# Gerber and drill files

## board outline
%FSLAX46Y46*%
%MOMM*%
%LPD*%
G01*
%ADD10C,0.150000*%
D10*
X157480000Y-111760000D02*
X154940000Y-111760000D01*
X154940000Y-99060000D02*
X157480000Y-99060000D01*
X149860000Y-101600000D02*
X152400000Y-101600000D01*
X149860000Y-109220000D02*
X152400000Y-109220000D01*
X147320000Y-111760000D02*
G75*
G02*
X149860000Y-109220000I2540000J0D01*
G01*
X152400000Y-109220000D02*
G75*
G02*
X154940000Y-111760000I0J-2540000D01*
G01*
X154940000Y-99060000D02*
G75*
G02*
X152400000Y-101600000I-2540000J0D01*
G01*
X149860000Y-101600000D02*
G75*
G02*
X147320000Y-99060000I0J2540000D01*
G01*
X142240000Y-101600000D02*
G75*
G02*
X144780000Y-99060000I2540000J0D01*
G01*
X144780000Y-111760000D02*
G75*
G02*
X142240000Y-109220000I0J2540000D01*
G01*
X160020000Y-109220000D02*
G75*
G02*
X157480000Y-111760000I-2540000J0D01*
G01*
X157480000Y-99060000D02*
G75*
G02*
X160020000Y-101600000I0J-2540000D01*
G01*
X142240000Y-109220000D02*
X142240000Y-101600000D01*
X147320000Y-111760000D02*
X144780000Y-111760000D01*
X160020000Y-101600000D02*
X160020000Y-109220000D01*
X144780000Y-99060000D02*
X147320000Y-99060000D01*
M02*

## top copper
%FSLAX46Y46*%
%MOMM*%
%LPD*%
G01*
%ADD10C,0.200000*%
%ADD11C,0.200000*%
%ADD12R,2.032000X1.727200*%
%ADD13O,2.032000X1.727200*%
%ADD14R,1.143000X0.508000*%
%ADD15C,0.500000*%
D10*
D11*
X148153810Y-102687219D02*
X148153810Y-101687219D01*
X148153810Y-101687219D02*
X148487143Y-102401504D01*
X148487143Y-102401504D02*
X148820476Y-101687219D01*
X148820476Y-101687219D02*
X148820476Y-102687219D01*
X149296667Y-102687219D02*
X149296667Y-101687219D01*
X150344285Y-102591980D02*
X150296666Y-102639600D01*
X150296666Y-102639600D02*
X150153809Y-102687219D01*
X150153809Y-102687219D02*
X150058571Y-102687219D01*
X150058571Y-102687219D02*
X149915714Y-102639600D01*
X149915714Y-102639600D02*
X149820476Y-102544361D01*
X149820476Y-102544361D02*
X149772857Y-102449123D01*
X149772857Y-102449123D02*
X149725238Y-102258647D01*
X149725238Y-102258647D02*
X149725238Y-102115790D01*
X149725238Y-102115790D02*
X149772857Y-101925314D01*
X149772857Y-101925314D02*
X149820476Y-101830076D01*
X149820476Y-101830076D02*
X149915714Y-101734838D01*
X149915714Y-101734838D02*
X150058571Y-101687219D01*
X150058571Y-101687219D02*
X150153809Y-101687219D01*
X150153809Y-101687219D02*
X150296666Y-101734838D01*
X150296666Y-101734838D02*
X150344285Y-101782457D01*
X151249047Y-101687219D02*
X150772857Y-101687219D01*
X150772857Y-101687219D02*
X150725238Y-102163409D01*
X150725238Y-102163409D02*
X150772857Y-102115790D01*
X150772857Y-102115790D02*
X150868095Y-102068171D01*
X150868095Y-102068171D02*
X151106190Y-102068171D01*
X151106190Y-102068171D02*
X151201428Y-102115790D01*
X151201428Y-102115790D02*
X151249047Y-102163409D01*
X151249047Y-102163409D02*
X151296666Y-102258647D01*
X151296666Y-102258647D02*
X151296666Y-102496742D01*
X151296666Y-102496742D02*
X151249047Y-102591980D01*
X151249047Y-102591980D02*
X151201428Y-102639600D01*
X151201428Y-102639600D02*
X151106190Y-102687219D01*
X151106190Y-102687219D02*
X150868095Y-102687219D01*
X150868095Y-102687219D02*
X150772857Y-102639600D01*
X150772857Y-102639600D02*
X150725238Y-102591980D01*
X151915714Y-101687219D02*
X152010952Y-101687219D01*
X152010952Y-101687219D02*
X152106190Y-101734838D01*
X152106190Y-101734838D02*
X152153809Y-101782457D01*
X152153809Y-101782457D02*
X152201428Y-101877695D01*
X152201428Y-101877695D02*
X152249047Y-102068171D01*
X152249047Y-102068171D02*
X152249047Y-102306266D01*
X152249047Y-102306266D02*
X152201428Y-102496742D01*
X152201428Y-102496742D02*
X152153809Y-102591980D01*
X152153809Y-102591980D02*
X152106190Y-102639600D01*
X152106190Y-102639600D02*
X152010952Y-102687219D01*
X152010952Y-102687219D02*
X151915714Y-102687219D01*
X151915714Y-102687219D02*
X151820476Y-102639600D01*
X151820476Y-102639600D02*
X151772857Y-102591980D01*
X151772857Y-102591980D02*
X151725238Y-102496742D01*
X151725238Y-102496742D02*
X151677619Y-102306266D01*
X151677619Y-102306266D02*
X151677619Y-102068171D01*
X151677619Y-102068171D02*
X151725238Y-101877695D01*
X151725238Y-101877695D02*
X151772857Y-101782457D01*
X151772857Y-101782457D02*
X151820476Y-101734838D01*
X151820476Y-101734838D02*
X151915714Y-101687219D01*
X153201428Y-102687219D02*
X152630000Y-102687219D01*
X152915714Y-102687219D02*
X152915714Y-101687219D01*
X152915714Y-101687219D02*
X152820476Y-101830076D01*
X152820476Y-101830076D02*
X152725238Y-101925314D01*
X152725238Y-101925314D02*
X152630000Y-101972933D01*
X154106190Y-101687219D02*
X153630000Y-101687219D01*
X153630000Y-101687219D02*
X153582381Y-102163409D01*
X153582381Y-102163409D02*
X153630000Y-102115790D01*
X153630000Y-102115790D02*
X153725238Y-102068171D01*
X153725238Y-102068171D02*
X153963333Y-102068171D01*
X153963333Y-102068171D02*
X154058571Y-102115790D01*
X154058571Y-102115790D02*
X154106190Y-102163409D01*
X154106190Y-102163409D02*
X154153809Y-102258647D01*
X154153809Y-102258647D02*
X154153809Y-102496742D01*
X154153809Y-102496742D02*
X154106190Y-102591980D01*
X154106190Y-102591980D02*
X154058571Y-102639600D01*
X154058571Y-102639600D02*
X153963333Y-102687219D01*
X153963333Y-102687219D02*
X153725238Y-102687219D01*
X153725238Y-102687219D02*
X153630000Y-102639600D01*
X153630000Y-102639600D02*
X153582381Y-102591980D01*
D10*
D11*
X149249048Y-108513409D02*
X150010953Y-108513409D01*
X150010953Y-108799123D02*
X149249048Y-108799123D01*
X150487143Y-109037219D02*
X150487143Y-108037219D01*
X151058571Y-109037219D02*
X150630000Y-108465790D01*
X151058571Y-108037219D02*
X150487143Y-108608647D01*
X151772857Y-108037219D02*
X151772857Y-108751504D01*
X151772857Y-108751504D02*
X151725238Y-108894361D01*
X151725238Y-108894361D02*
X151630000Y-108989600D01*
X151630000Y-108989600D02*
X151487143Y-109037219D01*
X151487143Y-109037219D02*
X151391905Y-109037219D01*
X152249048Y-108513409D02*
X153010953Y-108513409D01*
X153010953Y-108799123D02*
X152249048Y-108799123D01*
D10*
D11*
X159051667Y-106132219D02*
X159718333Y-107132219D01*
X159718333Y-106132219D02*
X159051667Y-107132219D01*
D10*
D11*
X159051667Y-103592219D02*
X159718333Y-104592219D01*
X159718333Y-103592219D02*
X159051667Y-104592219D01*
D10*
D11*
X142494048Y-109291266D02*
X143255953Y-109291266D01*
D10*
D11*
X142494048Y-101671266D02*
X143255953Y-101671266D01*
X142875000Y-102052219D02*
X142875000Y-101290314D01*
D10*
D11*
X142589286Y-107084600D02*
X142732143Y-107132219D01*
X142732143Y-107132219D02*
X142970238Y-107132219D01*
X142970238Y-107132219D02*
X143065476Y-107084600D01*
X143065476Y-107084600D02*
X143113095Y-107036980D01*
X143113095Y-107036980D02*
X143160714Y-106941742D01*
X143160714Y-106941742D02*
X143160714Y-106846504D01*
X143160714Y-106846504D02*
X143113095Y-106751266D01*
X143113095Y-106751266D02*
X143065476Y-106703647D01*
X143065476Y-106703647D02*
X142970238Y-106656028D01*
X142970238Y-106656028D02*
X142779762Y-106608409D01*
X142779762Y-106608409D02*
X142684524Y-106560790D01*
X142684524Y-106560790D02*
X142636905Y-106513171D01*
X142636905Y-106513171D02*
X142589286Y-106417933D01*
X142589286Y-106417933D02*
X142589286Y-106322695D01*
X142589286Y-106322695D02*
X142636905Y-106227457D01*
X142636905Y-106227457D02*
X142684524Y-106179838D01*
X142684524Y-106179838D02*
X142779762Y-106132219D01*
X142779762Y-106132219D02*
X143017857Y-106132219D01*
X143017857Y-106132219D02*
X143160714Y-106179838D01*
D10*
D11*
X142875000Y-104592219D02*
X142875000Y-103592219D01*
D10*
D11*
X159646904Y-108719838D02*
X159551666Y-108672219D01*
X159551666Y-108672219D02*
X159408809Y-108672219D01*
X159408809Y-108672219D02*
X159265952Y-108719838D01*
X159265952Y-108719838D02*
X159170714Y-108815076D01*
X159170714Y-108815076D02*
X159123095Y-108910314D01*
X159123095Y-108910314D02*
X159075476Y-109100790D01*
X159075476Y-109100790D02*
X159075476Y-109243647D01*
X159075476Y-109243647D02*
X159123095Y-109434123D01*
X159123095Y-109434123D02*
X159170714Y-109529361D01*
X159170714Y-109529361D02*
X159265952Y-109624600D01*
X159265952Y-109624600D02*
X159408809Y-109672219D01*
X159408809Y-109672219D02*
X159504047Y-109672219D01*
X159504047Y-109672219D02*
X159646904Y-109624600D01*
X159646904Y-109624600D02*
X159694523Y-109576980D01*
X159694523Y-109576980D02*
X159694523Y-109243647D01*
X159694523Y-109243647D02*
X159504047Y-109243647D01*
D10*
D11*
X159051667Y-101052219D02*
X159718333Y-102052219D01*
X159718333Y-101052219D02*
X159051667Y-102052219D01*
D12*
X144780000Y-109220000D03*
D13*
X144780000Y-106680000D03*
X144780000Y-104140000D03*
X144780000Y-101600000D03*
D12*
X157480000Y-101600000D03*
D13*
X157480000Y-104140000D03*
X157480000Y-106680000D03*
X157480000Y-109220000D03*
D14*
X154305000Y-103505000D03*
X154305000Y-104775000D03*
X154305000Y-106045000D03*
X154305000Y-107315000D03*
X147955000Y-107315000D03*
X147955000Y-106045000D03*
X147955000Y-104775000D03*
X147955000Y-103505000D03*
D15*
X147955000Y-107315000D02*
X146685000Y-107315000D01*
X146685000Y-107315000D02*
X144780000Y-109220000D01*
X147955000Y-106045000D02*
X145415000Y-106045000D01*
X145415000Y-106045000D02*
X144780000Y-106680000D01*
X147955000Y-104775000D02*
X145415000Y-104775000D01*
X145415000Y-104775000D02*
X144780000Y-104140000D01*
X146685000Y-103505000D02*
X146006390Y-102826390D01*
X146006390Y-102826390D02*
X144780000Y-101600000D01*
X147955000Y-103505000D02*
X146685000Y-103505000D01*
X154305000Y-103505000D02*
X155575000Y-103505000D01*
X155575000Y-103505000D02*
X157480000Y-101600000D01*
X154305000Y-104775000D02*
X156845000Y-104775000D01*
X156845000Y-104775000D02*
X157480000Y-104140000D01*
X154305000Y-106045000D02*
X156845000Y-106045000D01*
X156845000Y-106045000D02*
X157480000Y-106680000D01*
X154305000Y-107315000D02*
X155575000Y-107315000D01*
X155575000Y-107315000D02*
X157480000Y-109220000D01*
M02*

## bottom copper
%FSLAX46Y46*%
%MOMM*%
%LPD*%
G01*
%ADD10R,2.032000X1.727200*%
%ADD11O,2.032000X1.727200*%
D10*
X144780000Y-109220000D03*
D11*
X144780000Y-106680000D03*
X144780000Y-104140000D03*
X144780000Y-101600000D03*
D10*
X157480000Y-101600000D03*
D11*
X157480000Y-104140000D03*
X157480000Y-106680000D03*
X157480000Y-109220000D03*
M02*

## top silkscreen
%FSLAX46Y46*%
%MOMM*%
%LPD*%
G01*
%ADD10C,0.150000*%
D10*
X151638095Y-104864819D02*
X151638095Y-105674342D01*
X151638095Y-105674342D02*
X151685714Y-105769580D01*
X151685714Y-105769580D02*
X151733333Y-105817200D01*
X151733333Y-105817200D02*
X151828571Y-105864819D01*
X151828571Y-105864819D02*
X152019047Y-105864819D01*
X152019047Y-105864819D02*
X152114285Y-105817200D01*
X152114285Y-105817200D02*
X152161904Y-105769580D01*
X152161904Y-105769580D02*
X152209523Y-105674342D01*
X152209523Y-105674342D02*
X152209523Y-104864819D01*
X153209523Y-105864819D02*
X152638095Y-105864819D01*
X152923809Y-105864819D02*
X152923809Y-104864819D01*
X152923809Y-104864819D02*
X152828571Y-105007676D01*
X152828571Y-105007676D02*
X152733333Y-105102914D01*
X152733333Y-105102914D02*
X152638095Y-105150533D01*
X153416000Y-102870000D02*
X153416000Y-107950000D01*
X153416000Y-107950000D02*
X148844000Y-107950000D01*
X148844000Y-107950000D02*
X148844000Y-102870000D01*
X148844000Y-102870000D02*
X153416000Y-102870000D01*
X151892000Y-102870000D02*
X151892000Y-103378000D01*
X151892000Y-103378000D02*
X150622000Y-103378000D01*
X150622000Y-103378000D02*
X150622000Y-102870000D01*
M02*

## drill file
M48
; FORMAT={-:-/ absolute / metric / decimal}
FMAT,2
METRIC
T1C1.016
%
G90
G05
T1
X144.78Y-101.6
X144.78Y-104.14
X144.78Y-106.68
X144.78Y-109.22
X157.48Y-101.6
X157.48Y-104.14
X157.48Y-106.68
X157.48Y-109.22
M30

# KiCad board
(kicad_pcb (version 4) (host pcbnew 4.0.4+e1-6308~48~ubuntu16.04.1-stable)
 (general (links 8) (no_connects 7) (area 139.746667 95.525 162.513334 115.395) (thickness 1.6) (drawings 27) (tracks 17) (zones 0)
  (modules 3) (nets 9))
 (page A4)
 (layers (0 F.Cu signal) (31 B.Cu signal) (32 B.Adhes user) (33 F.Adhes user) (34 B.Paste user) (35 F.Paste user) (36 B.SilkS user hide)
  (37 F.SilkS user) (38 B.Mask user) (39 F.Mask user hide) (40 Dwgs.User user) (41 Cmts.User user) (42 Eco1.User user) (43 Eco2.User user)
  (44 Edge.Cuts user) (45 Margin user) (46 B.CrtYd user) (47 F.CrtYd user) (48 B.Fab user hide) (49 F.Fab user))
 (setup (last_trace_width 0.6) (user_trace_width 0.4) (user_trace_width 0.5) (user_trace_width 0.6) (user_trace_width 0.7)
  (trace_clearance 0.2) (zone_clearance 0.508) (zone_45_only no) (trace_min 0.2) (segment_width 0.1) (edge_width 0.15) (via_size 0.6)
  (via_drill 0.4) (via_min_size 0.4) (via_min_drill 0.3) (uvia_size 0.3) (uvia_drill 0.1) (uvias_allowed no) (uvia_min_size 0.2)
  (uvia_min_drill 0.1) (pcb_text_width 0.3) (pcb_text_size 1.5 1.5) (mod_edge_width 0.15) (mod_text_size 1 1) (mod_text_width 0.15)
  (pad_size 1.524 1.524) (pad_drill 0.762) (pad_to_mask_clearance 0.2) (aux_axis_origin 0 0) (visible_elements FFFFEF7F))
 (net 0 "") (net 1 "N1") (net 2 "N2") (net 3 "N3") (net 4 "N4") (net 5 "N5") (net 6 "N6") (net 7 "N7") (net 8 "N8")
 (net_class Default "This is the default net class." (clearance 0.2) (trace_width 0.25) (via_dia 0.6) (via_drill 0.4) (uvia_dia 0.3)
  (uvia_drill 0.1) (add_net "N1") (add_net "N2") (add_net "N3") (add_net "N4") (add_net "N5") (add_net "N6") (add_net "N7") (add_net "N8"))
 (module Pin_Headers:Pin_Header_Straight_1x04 (layer B.Cu) (at 144.78 109.22)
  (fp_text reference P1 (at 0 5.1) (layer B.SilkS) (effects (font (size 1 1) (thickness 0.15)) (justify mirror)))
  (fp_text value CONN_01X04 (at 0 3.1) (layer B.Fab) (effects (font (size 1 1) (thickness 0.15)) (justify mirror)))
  (pad 1 thru_hole rect (at 0 0) (size 2.032 1.7272) (drill 1.016) (layers *.Cu *.Mask) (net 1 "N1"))
  (pad 2 thru_hole oval (at 0 -2.54) (size 2.032 1.7272) (drill 1.016) (layers *.Cu *.Mask) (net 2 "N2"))
  (pad 3 thru_hole oval (at 0 -5.08) (size 2.032 1.7272) (drill 1.016) (layers *.Cu *.Mask) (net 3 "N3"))
  (pad 4 thru_hole oval (at 0 -7.62) (size 2.032 1.7272) (drill 1.016) (layers *.Cu *.Mask) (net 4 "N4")))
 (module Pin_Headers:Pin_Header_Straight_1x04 (layer B.Cu) (at 157.48 101.6 180)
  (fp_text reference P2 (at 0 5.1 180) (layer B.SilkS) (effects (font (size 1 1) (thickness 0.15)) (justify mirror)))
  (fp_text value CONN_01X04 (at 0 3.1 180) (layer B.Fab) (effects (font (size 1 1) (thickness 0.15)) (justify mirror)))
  (pad 1 thru_hole rect (at 0 0 180) (size 2.032 1.7272) (drill 1.016) (layers *.Cu *.Mask) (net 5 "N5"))
  (pad 2 thru_hole oval (at 0 -2.54 180) (size 2.032 1.7272) (drill 1.016) (layers *.Cu *.Mask) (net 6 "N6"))
  (pad 3 thru_hole oval (at 0 -5.08 180) (size 2.032 1.7272) (drill 1.016) (layers *.Cu *.Mask) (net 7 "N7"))
  (pad 4 thru_hole oval (at 0 -7.62 180) (size 2.032 1.7272) (drill 1.016) (layers *.Cu *.Mask) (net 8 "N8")))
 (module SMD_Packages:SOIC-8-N (layer F.Cu) (at 151.13 105.41 270)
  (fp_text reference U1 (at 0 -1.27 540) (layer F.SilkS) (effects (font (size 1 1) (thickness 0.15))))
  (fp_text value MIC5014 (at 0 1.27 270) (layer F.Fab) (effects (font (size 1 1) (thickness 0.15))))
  (fp_line (start -2.54 -2.286) (end 2.54 -2.286) (layer F.SilkS) (width 0.15))
  (fp_line (start 2.54 -2.286) (end 2.54 2.286) (layer F.SilkS) (width 0.15))
  (fp_line (start 2.54 2.286) (end -2.54 2.286) (layer F.SilkS) (width 0.15))
  (fp_line (start -2.54 2.286) (end -2.54 -2.286) (layer F.SilkS) (width 0.15))
  (fp_line (start -2.54 -0.762) (end -2.032 -0.762) (layer F.SilkS) (width 0.15))
  (fp_line (start -2.032 -0.762) (end -2.032 0.508) (layer F.SilkS) (width 0.15))
  (fp_line (start -2.032 0.508) (end -2.54 0.508) (layer F.SilkS) (width 0.15))
  (pad 8 smd rect (at -1.905 -3.175 270) (size 0.508 1.143) (layers F.Cu F.Paste F.Mask) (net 5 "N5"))
  (pad 7 smd rect (at -0.635 -3.175 270) (size 0.508 1.143) (layers F.Cu F.Paste F.Mask) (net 6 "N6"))
  (pad 6 smd rect (at 0.635 -3.175 270) (size 0.508 1.143) (layers F.Cu F.Paste F.Mask) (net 7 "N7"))
  (pad 5 smd rect (at 1.905 -3.175 270) (size 0.508 1.143) (layers F.Cu F.Paste F.Mask) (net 8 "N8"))
  (pad 4 smd rect (at 1.905 3.175 270) (size 0.508 1.143) (layers F.Cu F.Paste F.Mask) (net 1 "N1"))
  (pad 3 smd rect (at 0.635 3.175 270) (size 0.508 1.143) (layers F.Cu F.Paste F.Mask) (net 2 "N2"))
  (pad 2 smd rect (at -0.635 3.175 270) (size 0.508 1.143) (layers F.Cu F.Paste F.Mask) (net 3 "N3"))
  (pad 1 smd rect (at -1.905 3.175 270) (size 0.508 1.143) (layers F.Cu F.Paste F.Mask) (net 4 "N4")))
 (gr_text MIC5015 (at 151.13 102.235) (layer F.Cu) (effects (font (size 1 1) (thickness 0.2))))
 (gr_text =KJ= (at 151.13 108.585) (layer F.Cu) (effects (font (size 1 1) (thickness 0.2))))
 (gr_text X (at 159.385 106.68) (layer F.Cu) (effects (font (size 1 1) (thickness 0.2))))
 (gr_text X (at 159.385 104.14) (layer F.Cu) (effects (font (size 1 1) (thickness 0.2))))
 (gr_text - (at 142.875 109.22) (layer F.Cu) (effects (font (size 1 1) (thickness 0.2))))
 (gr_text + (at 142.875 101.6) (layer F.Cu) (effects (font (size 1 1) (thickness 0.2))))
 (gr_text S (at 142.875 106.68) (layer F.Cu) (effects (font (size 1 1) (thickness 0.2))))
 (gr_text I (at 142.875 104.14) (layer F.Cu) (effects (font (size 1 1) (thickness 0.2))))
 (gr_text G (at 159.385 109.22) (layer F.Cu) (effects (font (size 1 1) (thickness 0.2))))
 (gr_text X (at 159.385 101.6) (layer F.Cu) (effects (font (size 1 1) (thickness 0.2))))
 (gr_line (start 157.48 111.76) (end 154.94 111.76) (layer Edge.Cuts) (width 0.15))
 (gr_line (start 154.94 99.06) (end 157.48 99.06) (layer Edge.Cuts) (width 0.15))
 (gr_line (start 149.86 101.6) (end 152.4 101.6) (layer Edge.Cuts) (width 0.15))
 (gr_line (start 149.86 109.22) (end 152.4 109.22) (layer Edge.Cuts) (width 0.15))
 (gr_arc (start 149.86 111.76) (end 147.32 111.76) (angle 90) (layer Edge.Cuts) (width 0.15))
 (gr_arc (start 152.4 111.76) (end 152.4 109.22) (angle 90) (layer Edge.Cuts) (width 0.15))
 (gr_arc (start 152.4 99.06) (end 154.94 99.06) (angle 90) (layer Edge.Cuts) (width 0.15))
 (gr_arc (start 149.86 99.06) (end 149.86 101.6) (angle 90) (layer Edge.Cuts) (width 0.15))
 (gr_arc (start 144.78 101.6) (end 142.24 101.6) (angle 90) (layer Edge.Cuts) (width 0.15))
 (gr_arc (start 144.78 109.22) (end 144.78 111.76) (angle 90) (layer Edge.Cuts) (width 0.15))
 (gr_arc (start 157.48 109.22) (end 160.02 109.22) (angle 90) (layer Edge.Cuts) (width 0.15))
 (gr_arc (start 157.48 101.6) (end 157.48 99.06) (angle 90) (layer Edge.Cuts) (width 0.15))
 (gr_line (start 142.24 109.22) (end 142.24 101.6) (layer Edge.Cuts) (width 0.15))
 (gr_line (start 147.32 111.76) (end 144.78 111.76) (layer Edge.Cuts) (width 0.15))
 (gr_line (start 160.02 101.6) (end 160.02 109.22) (layer Edge.Cuts) (width 0.15))
 (gr_line (start 144.78 99.06) (end 147.32 99.06) (layer Edge.Cuts) (width 0.15))
 (segment (start 147.955 107.315) (end 146.685 107.315) (width 0.5) (layer F.Cu) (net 1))
 (segment (start 146.685 107.315) (end 144.78 109.22) (width 0.5) (layer F.Cu) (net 1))
 (segment (start 147.955 106.045) (end 145.415 106.045) (width 0.5) (layer F.Cu) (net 2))
 (segment (start 145.415 106.045) (end 144.78 106.68) (width 0.5) (layer F.Cu) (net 2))
 (segment (start 147.955 104.775) (end 145.415 104.775) (width 0.5) (layer F.Cu) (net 3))
 (segment (start 145.415 104.775) (end 144.78 104.14) (width 0.5) (layer F.Cu) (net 3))
 (segment (start 146.685 103.505) (end 146.00639 102.82639) (width 0.5) (layer F.Cu) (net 4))
 (segment (start 146.00639 102.82639) (end 144.78 101.6) (width 0.5) (layer F.Cu) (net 4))
 (segment (start 147.955 103.505) (end 146.685 103.505) (width 0.5) (layer F.Cu) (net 4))
 (segment (start 154.305 103.505) (end 155.575 103.505) (width 0.5) (layer F.Cu) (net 5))
 (segment (start 155.575 103.505) (end 157.48 101.6) (width 0.5) (layer F.Cu) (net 5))
 (segment (start 154.305 104.775) (end 156.845 104.775) (width 0.5) (layer F.Cu) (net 6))
 (segment (start 156.845 104.775) (end 157.48 104.14) (width 0.5) (layer F.Cu) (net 6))
 (segment (start 154.305 106.045) (end 156.845 106.045) (width 0.5) (layer F.Cu) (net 7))
 (segment (start 156.845 106.045) (end 157.48 106.68) (width 0.5) (layer F.Cu) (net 7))
 (segment (start 154.305 107.315) (end 155.575 107.315) (width 0.5) (layer F.Cu) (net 8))
 (segment (start 155.575 107.315) (end 157.48 109.22) (width 0.5) (layer F.Cu) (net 8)))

